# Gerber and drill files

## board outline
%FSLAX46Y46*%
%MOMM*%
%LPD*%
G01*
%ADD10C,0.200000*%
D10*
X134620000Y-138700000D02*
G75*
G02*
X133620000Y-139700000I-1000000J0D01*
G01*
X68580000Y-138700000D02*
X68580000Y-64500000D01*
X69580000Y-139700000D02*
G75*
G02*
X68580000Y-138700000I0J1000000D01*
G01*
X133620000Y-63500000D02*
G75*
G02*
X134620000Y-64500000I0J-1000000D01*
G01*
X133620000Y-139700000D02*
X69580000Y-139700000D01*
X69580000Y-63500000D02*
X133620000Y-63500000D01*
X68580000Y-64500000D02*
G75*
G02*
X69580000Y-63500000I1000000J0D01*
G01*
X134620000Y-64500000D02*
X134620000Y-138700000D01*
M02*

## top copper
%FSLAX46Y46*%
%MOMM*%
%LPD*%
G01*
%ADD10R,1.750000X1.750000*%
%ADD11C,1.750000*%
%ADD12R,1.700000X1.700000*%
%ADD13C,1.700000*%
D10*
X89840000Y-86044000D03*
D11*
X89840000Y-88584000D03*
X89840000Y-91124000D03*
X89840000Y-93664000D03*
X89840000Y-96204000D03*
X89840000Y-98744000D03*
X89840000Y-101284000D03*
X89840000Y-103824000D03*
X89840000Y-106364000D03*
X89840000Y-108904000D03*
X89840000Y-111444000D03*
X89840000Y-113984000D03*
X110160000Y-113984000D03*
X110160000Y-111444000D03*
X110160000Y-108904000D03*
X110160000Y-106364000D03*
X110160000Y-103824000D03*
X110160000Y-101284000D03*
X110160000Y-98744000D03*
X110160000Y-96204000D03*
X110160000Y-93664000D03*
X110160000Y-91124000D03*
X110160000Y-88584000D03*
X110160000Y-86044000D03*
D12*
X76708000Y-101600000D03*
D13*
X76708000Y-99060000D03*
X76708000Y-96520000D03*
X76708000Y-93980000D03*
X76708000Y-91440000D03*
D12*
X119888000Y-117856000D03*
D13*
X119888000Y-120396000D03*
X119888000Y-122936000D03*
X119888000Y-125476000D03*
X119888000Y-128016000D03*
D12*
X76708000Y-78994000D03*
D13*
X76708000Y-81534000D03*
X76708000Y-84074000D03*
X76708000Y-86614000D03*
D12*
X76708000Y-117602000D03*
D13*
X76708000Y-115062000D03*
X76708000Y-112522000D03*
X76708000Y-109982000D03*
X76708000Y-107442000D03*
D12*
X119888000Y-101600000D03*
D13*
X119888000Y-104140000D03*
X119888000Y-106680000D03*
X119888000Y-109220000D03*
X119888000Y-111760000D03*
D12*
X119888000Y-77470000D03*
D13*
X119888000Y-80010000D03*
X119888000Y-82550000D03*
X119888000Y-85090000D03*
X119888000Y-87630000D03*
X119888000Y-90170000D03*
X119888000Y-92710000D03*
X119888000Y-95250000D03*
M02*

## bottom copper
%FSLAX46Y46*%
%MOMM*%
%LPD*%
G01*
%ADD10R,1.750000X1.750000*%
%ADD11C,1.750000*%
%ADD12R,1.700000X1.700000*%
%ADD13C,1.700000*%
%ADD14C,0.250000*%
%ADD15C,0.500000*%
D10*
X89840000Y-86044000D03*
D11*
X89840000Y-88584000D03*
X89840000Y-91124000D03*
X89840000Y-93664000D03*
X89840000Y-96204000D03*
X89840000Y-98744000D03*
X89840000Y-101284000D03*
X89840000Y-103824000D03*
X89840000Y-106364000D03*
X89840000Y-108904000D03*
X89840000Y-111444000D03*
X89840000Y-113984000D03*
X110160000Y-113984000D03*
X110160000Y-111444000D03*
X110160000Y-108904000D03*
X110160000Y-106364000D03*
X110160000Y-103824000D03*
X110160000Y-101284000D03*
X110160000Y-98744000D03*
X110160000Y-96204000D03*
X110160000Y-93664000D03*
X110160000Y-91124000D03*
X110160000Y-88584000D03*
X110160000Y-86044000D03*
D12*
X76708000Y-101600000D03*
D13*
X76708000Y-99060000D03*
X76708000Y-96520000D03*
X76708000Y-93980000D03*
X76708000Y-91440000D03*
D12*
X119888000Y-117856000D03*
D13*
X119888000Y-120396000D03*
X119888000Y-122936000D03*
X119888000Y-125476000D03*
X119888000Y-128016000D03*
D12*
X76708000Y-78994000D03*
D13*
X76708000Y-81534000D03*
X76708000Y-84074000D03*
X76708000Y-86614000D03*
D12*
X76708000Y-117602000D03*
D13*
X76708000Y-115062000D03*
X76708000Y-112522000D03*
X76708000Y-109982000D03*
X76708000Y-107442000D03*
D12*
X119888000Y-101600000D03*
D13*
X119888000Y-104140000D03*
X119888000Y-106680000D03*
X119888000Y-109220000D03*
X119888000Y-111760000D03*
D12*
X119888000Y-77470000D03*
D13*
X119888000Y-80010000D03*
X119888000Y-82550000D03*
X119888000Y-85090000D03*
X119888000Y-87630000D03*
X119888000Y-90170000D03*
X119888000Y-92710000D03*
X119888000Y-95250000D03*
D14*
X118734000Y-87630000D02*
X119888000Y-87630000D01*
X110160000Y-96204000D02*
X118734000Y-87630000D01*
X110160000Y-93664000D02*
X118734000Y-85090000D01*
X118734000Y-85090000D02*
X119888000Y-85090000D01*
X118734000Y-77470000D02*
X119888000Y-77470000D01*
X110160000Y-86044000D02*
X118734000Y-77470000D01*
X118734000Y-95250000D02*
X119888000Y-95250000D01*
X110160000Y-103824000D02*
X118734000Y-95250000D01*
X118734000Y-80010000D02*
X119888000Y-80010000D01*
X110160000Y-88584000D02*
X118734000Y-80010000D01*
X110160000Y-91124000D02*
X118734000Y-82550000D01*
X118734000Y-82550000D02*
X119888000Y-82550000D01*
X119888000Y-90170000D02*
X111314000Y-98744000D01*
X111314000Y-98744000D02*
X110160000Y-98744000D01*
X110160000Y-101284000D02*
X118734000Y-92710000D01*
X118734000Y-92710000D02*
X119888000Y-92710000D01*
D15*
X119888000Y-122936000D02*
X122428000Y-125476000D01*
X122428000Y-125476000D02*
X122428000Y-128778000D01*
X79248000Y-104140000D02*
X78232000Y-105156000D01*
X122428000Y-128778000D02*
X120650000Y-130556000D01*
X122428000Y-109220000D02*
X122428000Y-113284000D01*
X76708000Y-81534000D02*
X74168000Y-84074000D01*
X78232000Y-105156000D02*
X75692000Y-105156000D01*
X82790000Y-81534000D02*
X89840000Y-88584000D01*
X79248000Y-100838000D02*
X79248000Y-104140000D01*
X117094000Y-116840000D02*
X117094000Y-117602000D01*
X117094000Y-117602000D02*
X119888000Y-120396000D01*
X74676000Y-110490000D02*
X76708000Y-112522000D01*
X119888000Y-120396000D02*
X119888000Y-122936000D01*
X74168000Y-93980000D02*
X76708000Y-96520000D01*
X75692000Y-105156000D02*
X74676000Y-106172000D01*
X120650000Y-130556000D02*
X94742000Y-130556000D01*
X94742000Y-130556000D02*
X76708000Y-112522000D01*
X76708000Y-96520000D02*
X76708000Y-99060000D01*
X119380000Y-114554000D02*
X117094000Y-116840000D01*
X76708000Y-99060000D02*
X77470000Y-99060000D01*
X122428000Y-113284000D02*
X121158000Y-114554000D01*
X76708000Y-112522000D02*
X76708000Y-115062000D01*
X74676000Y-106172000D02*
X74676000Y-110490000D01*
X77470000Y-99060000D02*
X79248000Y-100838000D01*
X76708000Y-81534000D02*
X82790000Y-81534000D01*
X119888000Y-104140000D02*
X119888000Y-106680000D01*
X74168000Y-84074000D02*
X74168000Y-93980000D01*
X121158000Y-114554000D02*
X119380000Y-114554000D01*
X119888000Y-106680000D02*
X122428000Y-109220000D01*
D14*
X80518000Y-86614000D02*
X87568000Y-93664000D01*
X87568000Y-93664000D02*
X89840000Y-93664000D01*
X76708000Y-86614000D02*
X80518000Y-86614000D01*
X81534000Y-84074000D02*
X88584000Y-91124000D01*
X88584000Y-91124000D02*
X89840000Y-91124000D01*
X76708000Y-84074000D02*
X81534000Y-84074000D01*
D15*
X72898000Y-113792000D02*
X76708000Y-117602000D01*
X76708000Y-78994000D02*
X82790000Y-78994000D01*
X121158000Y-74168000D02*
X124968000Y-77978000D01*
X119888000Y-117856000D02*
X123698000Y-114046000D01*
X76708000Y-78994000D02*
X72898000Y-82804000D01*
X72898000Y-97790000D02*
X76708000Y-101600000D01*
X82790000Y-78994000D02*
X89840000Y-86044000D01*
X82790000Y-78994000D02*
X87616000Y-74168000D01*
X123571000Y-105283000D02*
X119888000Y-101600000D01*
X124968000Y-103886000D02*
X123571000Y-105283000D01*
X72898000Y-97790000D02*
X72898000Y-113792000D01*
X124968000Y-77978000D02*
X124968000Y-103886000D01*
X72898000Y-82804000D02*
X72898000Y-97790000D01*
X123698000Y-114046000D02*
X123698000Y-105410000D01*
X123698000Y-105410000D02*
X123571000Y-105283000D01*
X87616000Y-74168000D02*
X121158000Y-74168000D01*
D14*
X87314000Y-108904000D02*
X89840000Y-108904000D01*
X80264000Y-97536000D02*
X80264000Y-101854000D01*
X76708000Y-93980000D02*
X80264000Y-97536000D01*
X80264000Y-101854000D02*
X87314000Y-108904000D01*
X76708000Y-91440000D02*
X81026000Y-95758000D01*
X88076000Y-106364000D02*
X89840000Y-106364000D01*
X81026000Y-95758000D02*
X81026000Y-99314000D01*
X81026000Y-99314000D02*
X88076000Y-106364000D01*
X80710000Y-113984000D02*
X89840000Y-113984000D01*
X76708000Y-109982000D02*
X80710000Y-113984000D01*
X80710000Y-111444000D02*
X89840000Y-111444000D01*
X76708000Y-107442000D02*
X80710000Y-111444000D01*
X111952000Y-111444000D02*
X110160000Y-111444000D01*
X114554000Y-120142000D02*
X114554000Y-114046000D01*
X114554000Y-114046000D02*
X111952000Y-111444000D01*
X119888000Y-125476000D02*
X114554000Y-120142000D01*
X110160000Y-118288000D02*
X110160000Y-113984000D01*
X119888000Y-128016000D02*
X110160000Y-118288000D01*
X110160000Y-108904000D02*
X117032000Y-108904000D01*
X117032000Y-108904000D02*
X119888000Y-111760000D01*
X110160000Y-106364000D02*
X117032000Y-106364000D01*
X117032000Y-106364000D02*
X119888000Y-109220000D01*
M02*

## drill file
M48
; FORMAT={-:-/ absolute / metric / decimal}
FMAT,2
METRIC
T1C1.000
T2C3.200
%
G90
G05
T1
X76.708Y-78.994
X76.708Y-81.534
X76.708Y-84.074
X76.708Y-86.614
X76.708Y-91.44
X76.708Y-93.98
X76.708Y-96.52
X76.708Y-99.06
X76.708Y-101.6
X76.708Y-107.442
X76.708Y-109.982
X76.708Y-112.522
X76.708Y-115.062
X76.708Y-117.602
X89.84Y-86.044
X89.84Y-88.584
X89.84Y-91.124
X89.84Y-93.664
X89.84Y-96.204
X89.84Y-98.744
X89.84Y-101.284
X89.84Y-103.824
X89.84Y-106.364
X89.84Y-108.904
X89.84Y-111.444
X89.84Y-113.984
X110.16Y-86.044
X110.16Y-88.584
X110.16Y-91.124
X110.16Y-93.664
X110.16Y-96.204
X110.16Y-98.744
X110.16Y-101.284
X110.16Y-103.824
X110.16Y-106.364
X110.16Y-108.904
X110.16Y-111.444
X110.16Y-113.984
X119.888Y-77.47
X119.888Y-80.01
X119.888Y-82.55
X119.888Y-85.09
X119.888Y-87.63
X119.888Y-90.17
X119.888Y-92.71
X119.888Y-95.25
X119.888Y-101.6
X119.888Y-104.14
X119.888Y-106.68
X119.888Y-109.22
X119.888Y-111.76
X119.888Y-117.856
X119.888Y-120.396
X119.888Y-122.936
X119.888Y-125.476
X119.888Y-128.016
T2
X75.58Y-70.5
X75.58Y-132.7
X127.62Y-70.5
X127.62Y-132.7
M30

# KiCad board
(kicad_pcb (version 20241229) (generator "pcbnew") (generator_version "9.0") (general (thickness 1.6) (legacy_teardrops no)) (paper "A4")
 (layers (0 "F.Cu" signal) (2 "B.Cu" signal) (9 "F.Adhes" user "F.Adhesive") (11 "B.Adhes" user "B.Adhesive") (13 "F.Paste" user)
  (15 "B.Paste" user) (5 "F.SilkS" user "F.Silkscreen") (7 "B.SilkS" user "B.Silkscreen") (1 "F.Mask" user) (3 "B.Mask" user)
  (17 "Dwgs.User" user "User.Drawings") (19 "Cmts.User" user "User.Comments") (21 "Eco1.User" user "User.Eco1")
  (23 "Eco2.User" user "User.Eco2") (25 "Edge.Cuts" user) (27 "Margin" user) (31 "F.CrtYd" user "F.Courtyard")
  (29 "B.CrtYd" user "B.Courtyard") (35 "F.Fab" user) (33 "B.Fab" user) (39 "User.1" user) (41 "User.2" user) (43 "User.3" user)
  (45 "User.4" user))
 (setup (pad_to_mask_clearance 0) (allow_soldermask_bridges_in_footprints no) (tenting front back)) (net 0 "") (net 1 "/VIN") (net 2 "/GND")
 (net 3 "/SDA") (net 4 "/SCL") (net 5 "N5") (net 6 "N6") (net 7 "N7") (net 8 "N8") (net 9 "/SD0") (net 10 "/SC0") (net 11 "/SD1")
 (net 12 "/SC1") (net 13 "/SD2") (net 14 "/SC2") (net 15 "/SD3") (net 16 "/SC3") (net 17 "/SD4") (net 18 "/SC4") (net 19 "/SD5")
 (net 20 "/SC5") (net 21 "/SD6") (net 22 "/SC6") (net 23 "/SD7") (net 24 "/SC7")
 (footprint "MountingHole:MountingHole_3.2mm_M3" (layer "F.Cu") (at 127.62 70.5)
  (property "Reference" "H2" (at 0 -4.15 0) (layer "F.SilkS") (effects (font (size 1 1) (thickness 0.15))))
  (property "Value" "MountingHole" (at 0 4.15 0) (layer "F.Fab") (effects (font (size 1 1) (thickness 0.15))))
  (pad "" np_thru_hole circle (at 0 0) (size 3.2 3.2) (drill 3.2) (layers "*.Cu" "*.Mask")))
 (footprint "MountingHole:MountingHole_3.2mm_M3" (layer "F.Cu") (at 127.62 132.7)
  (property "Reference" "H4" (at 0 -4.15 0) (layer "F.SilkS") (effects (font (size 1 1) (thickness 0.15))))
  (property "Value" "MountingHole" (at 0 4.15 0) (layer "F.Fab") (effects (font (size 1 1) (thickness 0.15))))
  (pad "" np_thru_hole circle (at 0 0) (size 3.2 3.2) (drill 3.2) (layers "*.Cu" "*.Mask")))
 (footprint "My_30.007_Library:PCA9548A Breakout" (layer "F.Cu") (at 89.84 86.044)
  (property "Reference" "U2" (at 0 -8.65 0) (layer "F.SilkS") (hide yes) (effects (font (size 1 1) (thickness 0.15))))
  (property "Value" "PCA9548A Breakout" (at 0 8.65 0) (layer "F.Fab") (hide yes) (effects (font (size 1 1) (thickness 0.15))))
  (pad "1" thru_hole rect (at 0 0) (size 1.75 1.75) (drill 1) (layers "*.Cu" "*.Mask") (remove_unused_layers no) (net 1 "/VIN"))
  (pad "2" thru_hole circle (at 0 2.54) (size 1.75 1.75) (drill 1) (layers "*.Cu" "*.Mask") (remove_unused_layers no) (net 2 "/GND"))
  (pad "3" thru_hole circle (at 0 5.08) (size 1.75 1.75) (drill 1) (layers "*.Cu" "*.Mask") (remove_unused_layers no) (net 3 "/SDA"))
  (pad "4" thru_hole circle (at 0 7.62) (size 1.75 1.75) (drill 1) (layers "*.Cu" "*.Mask") (remove_unused_layers no) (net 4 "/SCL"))
  (pad "5" thru_hole circle (at 0 10.16) (size 1.75 1.75) (drill 1) (layers "*.Cu" "*.Mask") (remove_unused_layers no) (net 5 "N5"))
  (pad "6" thru_hole circle (at 0 12.7) (size 1.75 1.75) (drill 1) (layers "*.Cu" "*.Mask") (remove_unused_layers no) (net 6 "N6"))
  (pad "7" thru_hole circle (at 0 15.24) (size 1.75 1.75) (drill 1) (layers "*.Cu" "*.Mask") (remove_unused_layers no) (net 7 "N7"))
  (pad "8" thru_hole circle (at 0 17.78) (size 1.75 1.75) (drill 1) (layers "*.Cu" "*.Mask") (remove_unused_layers no) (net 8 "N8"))
  (pad "9" thru_hole circle (at 0 20.32) (size 1.75 1.75) (drill 1) (layers "*.Cu" "*.Mask") (remove_unused_layers no) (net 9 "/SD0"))
  (pad "10" thru_hole circle (at 0 22.86) (size 1.75 1.75) (drill 1) (layers "*.Cu" "*.Mask") (remove_unused_layers no) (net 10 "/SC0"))
  (pad "11" thru_hole circle (at 0 25.4) (size 1.75 1.75) (drill 1) (layers "*.Cu" "*.Mask") (remove_unused_layers no) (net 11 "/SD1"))
  (pad "12" thru_hole circle (at 0 27.94) (size 1.75 1.75) (drill 1) (layers "*.Cu" "*.Mask") (remove_unused_layers no) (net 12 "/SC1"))
  (pad "13" thru_hole circle (at 20.32 27.94) (size 1.75 1.75) (drill 1) (layers "*.Cu" "*.Mask") (remove_unused_layers no) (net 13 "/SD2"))
  (pad "14" thru_hole circle (at 20.32 25.4) (size 1.75 1.75) (drill 1) (layers "*.Cu" "*.Mask") (remove_unused_layers no) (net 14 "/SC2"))
  (pad "15" thru_hole circle (at 20.32 22.86) (size 1.75 1.75) (drill 1) (layers "*.Cu" "*.Mask") (remove_unused_layers no) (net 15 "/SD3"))
  (pad "16" thru_hole circle (at 20.32 20.32) (size 1.75 1.75) (drill 1) (layers "*.Cu" "*.Mask") (remove_unused_layers no) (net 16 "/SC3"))
  (pad "17" thru_hole circle (at 20.32 17.78) (size 1.75 1.75) (drill 1) (layers "*.Cu" "*.Mask") (remove_unused_layers no) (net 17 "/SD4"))
  (pad "18" thru_hole circle (at 20.32 15.24) (size 1.75 1.75) (drill 1) (layers "*.Cu" "*.Mask") (remove_unused_layers no) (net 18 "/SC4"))
  (pad "19" thru_hole circle (at 20.32 12.7) (size 1.75 1.75) (drill 1) (layers "*.Cu" "*.Mask") (remove_unused_layers no) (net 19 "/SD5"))
  (pad "20" thru_hole circle (at 20.32 10.16) (size 1.75 1.75) (drill 1) (layers "*.Cu" "*.Mask") (remove_unused_layers no) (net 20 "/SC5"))
  (pad "21" thru_hole circle (at 20.32 7.62) (size 1.75 1.75) (drill 1) (layers "*.Cu" "*.Mask") (remove_unused_layers no) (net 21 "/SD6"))
  (pad "22" thru_hole circle (at 20.32 5.08) (size 1.75 1.75) (drill 1) (layers "*.Cu" "*.Mask") (remove_unused_layers no) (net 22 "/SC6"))
  (pad "23" thru_hole circle (at 20.32 2.54) (size 1.75 1.75) (drill 1) (layers "*.Cu" "*.Mask") (remove_unused_layers no) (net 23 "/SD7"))
  (pad "24" thru_hole circle (at 20.32 0) (size 1.75 1.75) (drill 1) (layers "*.Cu" "*.Mask") (remove_unused_layers no) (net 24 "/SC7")))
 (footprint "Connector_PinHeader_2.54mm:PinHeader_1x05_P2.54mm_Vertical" (layer "F.Cu") (at 76.708 101.6 180)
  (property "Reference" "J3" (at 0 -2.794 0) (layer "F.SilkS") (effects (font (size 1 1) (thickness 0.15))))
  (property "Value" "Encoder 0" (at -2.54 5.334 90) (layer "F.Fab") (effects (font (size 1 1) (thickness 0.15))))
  (pad "1" thru_hole rect (at 0 0 180) (size 1.7 1.7) (drill 1) (layers "*.Cu" "*.Mask") (remove_unused_layers no) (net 1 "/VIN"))
  (pad "2" thru_hole circle (at 0 2.54 180) (size 1.7 1.7) (drill 1) (layers "*.Cu" "*.Mask") (remove_unused_layers no) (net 2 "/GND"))
  (pad "3" thru_hole circle (at 0 5.08 180) (size 1.7 1.7) (drill 1) (layers "*.Cu" "*.Mask") (remove_unused_layers no) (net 2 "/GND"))
  (pad "4" thru_hole circle (at 0 7.62 180) (size 1.7 1.7) (drill 1) (layers "*.Cu" "*.Mask") (remove_unused_layers no) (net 10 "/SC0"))
  (pad "5" thru_hole circle (at 0 10.16 180) (size 1.7 1.7) (drill 1) (layers "*.Cu" "*.Mask") (remove_unused_layers no) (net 9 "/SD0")))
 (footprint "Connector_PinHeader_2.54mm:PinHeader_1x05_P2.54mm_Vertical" (layer "F.Cu") (at 119.888 117.856)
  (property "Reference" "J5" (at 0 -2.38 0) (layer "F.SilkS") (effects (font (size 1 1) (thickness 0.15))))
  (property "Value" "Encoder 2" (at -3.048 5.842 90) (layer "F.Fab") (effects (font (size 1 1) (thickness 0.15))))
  (pad "1" thru_hole rect (at 0 0) (size 1.7 1.7) (drill 1) (layers "*.Cu" "*.Mask") (remove_unused_layers no) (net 1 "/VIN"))
  (pad "2" thru_hole circle (at 0 2.54) (size 1.7 1.7) (drill 1) (layers "*.Cu" "*.Mask") (remove_unused_layers no) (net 2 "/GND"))
  (pad "3" thru_hole circle (at 0 5.08) (size 1.7 1.7) (drill 1) (layers "*.Cu" "*.Mask") (remove_unused_layers no) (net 2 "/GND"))
  (pad "4" thru_hole circle (at 0 7.62) (size 1.7 1.7) (drill 1) (layers "*.Cu" "*.Mask") (remove_unused_layers no) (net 14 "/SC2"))
  (pad "5" thru_hole circle (at 0 10.16) (size 1.7 1.7) (drill 1) (layers "*.Cu" "*.Mask") (remove_unused_layers no) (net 13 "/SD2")))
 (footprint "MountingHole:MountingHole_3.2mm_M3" (layer "F.Cu") (at 75.58 132.7)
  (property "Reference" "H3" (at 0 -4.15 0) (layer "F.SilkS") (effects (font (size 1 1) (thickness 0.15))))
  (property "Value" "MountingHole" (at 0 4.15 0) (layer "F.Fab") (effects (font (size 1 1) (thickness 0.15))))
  (pad "" np_thru_hole circle (at 0 0) (size 3.2 3.2) (drill 3.2) (layers "*.Cu" "*.Mask")))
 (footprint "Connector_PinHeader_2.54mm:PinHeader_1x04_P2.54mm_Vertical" (layer "F.Cu") (at 76.708 78.994)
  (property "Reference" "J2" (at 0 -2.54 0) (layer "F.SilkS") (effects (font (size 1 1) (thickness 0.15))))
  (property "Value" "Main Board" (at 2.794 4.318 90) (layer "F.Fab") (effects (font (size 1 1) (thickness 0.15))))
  (pad "1" thru_hole rect (at 0 0) (size 1.7 1.7) (drill 1) (layers "*.Cu" "*.Mask") (remove_unused_layers no) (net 1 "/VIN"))
  (pad "2" thru_hole circle (at 0 2.54) (size 1.7 1.7) (drill 1) (layers "*.Cu" "*.Mask") (remove_unused_layers no) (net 2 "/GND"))
  (pad "3" thru_hole circle (at 0 5.08) (size 1.7 1.7) (drill 1) (layers "*.Cu" "*.Mask") (remove_unused_layers no) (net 3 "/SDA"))
  (pad "4" thru_hole circle (at 0 7.62) (size 1.7 1.7) (drill 1) (layers "*.Cu" "*.Mask") (remove_unused_layers no) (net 4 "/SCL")))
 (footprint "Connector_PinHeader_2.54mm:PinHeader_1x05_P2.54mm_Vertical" (layer "F.Cu") (at 76.708 117.602 180)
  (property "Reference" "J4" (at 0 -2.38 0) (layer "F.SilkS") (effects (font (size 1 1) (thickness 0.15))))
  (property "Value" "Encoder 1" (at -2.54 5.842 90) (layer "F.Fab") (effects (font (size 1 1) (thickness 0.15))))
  (pad "1" thru_hole rect (at 0 0 180) (size 1.7 1.7) (drill 1) (layers "*.Cu" "*.Mask") (remove_unused_layers no) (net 1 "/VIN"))
  (pad "2" thru_hole circle (at 0 2.54 180) (size 1.7 1.7) (drill 1) (layers "*.Cu" "*.Mask") (remove_unused_layers no) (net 2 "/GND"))
  (pad "3" thru_hole circle (at 0 5.08 180) (size 1.7 1.7) (drill 1) (layers "*.Cu" "*.Mask") (remove_unused_layers no) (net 2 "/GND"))
  (pad "4" thru_hole circle (at 0 7.62 180) (size 1.7 1.7) (drill 1) (layers "*.Cu" "*.Mask") (remove_unused_layers no) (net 12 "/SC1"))
  (pad "5" thru_hole circle (at 0 10.16 180) (size 1.7 1.7) (drill 1) (layers "*.Cu" "*.Mask") (remove_unused_layers no) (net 11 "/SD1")))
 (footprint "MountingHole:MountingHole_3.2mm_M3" (layer "F.Cu") (at 75.58 70.5)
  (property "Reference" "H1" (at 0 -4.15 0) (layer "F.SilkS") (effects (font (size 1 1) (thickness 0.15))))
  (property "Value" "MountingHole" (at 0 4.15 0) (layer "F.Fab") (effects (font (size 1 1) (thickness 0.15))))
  (pad "" np_thru_hole circle (at 0 0) (size 3.2 3.2) (drill 3.2) (layers "*.Cu" "*.Mask")))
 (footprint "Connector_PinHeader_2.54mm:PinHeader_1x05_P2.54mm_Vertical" (layer "F.Cu") (at 119.888 101.6)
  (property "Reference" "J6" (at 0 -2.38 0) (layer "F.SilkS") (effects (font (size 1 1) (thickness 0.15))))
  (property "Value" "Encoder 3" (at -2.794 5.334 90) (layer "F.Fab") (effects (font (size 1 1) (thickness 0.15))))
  (pad "1" thru_hole rect (at 0 0) (size 1.7 1.7) (drill 1) (layers "*.Cu" "*.Mask") (remove_unused_layers no) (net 1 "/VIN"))
  (pad "2" thru_hole circle (at 0 2.54) (size 1.7 1.7) (drill 1) (layers "*.Cu" "*.Mask") (remove_unused_layers no) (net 2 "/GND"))
  (pad "3" thru_hole circle (at 0 5.08) (size 1.7 1.7) (drill 1) (layers "*.Cu" "*.Mask") (remove_unused_layers no) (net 2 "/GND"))
  (pad "4" thru_hole circle (at 0 7.62) (size 1.7 1.7) (drill 1) (layers "*.Cu" "*.Mask") (remove_unused_layers no) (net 16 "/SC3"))
  (pad "5" thru_hole circle (at 0 10.16) (size 1.7 1.7) (drill 1) (layers "*.Cu" "*.Mask") (remove_unused_layers no) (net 15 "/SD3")))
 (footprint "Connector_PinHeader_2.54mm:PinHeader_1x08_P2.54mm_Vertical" (layer "F.Cu") (at 119.888 77.47)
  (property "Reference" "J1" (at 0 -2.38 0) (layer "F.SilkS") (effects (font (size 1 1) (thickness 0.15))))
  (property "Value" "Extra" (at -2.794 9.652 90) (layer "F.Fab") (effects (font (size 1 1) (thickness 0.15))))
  (pad "1" thru_hole rect (at 0 0) (size 1.7 1.7) (drill 1) (layers "*.Cu" "*.Mask") (remove_unused_layers no) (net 24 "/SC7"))
  (pad "2" thru_hole circle (at 0 2.54) (size 1.7 1.7) (drill 1) (layers "*.Cu" "*.Mask") (remove_unused_layers no) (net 23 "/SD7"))
  (pad "3" thru_hole circle (at 0 5.08) (size 1.7 1.7) (drill 1) (layers "*.Cu" "*.Mask") (remove_unused_layers no) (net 22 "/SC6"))
  (pad "4" thru_hole circle (at 0 7.62) (size 1.7 1.7) (drill 1) (layers "*.Cu" "*.Mask") (remove_unused_layers no) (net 21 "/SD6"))
  (pad "5" thru_hole circle (at 0 10.16) (size 1.7 1.7) (drill 1) (layers "*.Cu" "*.Mask") (remove_unused_layers no) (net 20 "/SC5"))
  (pad "6" thru_hole circle (at 0 12.7) (size 1.7 1.7) (drill 1) (layers "*.Cu" "*.Mask") (remove_unused_layers no) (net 19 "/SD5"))
  (pad "7" thru_hole circle (at 0 15.24) (size 1.7 1.7) (drill 1) (layers "*.Cu" "*.Mask") (remove_unused_layers no) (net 18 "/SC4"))
  (pad "8" thru_hole circle (at 0 17.78) (size 1.7 1.7) (drill 1) (layers "*.Cu" "*.Mask") (remove_unused_layers no) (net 17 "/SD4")))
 (gr_arc (start 134.62 138.7) (mid 134.327107 139.407107) (end 133.62 139.7) (stroke (width 0.2) (type default)) (layer "Edge.Cuts"))
 (gr_line (start 68.58 138.7) (end 68.58 64.5) (stroke (width 0.2) (type default)) (layer "Edge.Cuts"))
 (gr_arc (start 69.58 139.7) (mid 68.872893 139.407107) (end 68.58 138.7) (stroke (width 0.2) (type default)) (layer "Edge.Cuts"))
 (gr_arc (start 133.62 63.5) (mid 134.327107 63.792893) (end 134.62 64.5) (stroke (width 0.2) (type default)) (layer "Edge.Cuts"))
 (gr_line (start 133.62 139.7) (end 69.58 139.7) (stroke (width 0.2) (type default)) (layer "Edge.Cuts"))
 (gr_line (start 69.58 63.5) (end 133.62 63.5) (stroke (width 0.2) (type default)) (layer "Edge.Cuts"))
 (gr_arc (start 68.58 64.5) (mid 68.872893 63.792893) (end 69.58 63.5) (stroke (width 0.2) (type default)) (layer "Edge.Cuts"))
 (gr_line (start 134.62 64.5) (end 134.62 138.7) (stroke (width 0.2) (type default)) (layer "Edge.Cuts"))
 (segment (start 118.734 87.63) (end 119.888 87.63) (width 0.25) (layer "B.Cu") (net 20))
 (segment (start 110.16 96.204) (end 118.734 87.63) (width 0.25) (layer "B.Cu") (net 20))
 (segment (start 110.16 93.664) (end 118.734 85.09) (width 0.25) (layer "B.Cu") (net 21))
 (segment (start 118.734 85.09) (end 119.888 85.09) (width 0.25) (layer "B.Cu") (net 21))
 (segment (start 118.734 77.47) (end 119.888 77.47) (width 0.25) (layer "B.Cu") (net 24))
 (segment (start 110.16 86.044) (end 118.734 77.47) (width 0.25) (layer "B.Cu") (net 24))
 (segment (start 118.734 95.25) (end 119.888 95.25) (width 0.25) (layer "B.Cu") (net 17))
 (segment (start 110.16 103.824) (end 118.734 95.25) (width 0.25) (layer "B.Cu") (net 17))
 (segment (start 118.734 80.01) (end 119.888 80.01) (width 0.25) (layer "B.Cu") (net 23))
 (segment (start 110.16 88.584) (end 118.734 80.01) (width 0.25) (layer "B.Cu") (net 23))
 (segment (start 110.16 91.124) (end 118.734 82.55) (width 0.25) (layer "B.Cu") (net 22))
 (segment (start 118.734 82.55) (end 119.888 82.55) (width 0.25) (layer "B.Cu") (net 22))
 (segment (start 119.888 90.17) (end 111.314 98.744) (width 0.25) (layer "B.Cu") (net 19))
 (segment (start 111.314 98.744) (end 110.16 98.744) (width 0.25) (layer "B.Cu") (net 19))
 (segment (start 110.16 101.284) (end 118.734 92.71) (width 0.25) (layer "B.Cu") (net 18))
 (segment (start 118.734 92.71) (end 119.888 92.71) (width 0.25) (layer "B.Cu") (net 18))
 (segment (start 119.888 122.936) (end 122.428 125.476) (width 0.5) (layer "B.Cu") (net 2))
 (segment (start 122.428 125.476) (end 122.428 128.778) (width 0.5) (layer "B.Cu") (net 2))
 (segment (start 79.248 104.14) (end 78.232 105.156) (width 0.5) (layer "B.Cu") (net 2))
 (segment (start 122.428 128.778) (end 120.65 130.556) (width 0.5) (layer "B.Cu") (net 2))
 (segment (start 122.428 109.22) (end 122.428 113.284) (width 0.5) (layer "B.Cu") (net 2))
 (segment (start 76.708 81.534) (end 74.168 84.074) (width 0.5) (layer "B.Cu") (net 2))
 (segment (start 78.232 105.156) (end 75.692 105.156) (width 0.5) (layer "B.Cu") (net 2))
 (segment (start 82.79 81.534) (end 89.84 88.584) (width 0.5) (layer "B.Cu") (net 2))
 (segment (start 79.248 100.838) (end 79.248 104.14) (width 0.5) (layer "B.Cu") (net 2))
 (segment (start 117.094 116.84) (end 117.094 117.602) (width 0.5) (layer "B.Cu") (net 2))
 (segment (start 117.094 117.602) (end 119.888 120.396) (width 0.5) (layer "B.Cu") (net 2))
 (segment (start 74.676 110.49) (end 76.708 112.522) (width 0.5) (layer "B.Cu") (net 2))
 (segment (start 119.888 120.396) (end 119.888 122.936) (width 0.5) (layer "B.Cu") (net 2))
 (segment (start 74.168 93.98) (end 76.708 96.52) (width 0.5) (layer "B.Cu") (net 2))
 (segment (start 75.692 105.156) (end 74.676 106.172) (width 0.5) (layer "B.Cu") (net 2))
 (segment (start 120.65 130.556) (end 94.742 130.556) (width 0.5) (layer "B.Cu") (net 2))
 (segment (start 94.742 130.556) (end 76.708 112.522) (width 0.5) (layer "B.Cu") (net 2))
 (segment (start 76.708 96.52) (end 76.708 99.06) (width 0.5) (layer "B.Cu") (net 2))
 (segment (start 119.38 114.554) (end 117.094 116.84) (width 0.5) (layer "B.Cu") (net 2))
 (segment (start 76.708 99.06) (end 77.47 99.06) (width 0.5) (layer "B.Cu") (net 2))
 (segment (start 122.428 113.284) (end 121.158 114.554) (width 0.5) (layer "B.Cu") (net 2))
 (segment (start 76.708 112.522) (end 76.708 115.062) (width 0.5) (layer "B.Cu") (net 2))
 (segment (start 74.676 106.172) (end 74.676 110.49) (width 0.5) (layer "B.Cu") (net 2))
 (segment (start 77.47 99.06) (end 79.248 100.838) (width 0.5) (layer "B.Cu") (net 2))
 (segment (start 76.708 81.534) (end 82.79 81.534) (width 0.5) (layer "B.Cu") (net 2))
 (segment (start 119.888 104.14) (end 119.888 106.68) (width 0.5) (layer "B.Cu") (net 2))
 (segment (start 74.168 84.074) (end 74.168 93.98) (width 0.5) (layer "B.Cu") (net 2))
 (segment (start 121.158 114.554) (end 119.38 114.554) (width 0.5) (layer "B.Cu") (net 2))
 (segment (start 119.888 106.68) (end 122.428 109.22) (width 0.5) (layer "B.Cu") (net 2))
 (segment (start 80.518 86.614) (end 87.568 93.664) (width 0.25) (layer "B.Cu") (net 4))
 (segment (start 87.568 93.664) (end 89.84 93.664) (width 0.25) (layer "B.Cu") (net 4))
 (segment (start 76.708 86.614) (end 80.518 86.614) (width 0.25) (layer "B.Cu") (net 4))
 (segment (start 81.534 84.074) (end 88.584 91.124) (width 0.25) (layer "B.Cu") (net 3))
 (segment (start 88.584 91.124) (end 89.84 91.124) (width 0.25) (layer "B.Cu") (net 3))
 (segment (start 76.708 84.074) (end 81.534 84.074) (width 0.25) (layer "B.Cu") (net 3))
 (segment (start 72.898 113.792) (end 76.708 117.602) (width 0.5) (layer "B.Cu") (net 1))
 (segment (start 76.708 78.994) (end 82.79 78.994) (width 0.5) (layer "B.Cu") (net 1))
 (segment (start 121.158 74.168) (end 124.968 77.978) (width 0.5) (layer "B.Cu") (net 1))
 (segment (start 119.888 117.856) (end 123.698 114.046) (width 0.5) (layer "B.Cu") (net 1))
 (segment (start 76.708 78.994) (end 72.898 82.804) (width 0.5) (layer "B.Cu") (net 1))
 (segment (start 72.898 97.79) (end 76.708 101.6) (width 0.5) (layer "B.Cu") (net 1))
 (segment (start 82.79 78.994) (end 89.84 86.044) (width 0.5) (layer "B.Cu") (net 1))
 (segment (start 82.79 78.994) (end 87.616 74.168) (width 0.5) (layer "B.Cu") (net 1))
 (segment (start 123.571 105.283) (end 119.888 101.6) (width 0.5) (layer "B.Cu") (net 1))
 (segment (start 124.968 103.886) (end 123.571 105.283) (width 0.5) (layer "B.Cu") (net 1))
 (segment (start 72.898 97.79) (end 72.898 113.792) (width 0.5) (layer "B.Cu") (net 1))
 (segment (start 124.968 77.978) (end 124.968 103.886) (width 0.5) (layer "B.Cu") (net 1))
 (segment (start 72.898 82.804) (end 72.898 97.79) (width 0.5) (layer "B.Cu") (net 1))
 (segment (start 123.698 114.046) (end 123.698 105.41) (width 0.5) (layer "B.Cu") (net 1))
 (segment (start 123.698 105.41) (end 123.571 105.283) (width 0.5) (layer "B.Cu") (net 1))
 (segment (start 87.616 74.168) (end 121.158 74.168) (width 0.5) (layer "B.Cu") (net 1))
 (segment (start 87.314 108.904) (end 89.84 108.904) (width 0.25) (layer "B.Cu") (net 10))
 (segment (start 80.264 97.536) (end 80.264 101.854) (width 0.25) (layer "B.Cu") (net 10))
 (segment (start 76.708 93.98) (end 80.264 97.536) (width 0.25) (layer "B.Cu") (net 10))
 (segment (start 80.264 101.854) (end 87.314 108.904) (width 0.25) (layer "B.Cu") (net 10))
 (segment (start 76.708 91.44) (end 81.026 95.758) (width 0.25) (layer "B.Cu") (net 9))
 (segment (start 88.076 106.364) (end 89.84 106.364) (width 0.25) (layer "B.Cu") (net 9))
 (segment (start 81.026 95.758) (end 81.026 99.314) (width 0.25) (layer "B.Cu") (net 9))
 (segment (start 81.026 99.314) (end 88.076 106.364) (width 0.25) (layer "B.Cu") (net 9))
 (segment (start 80.71 113.984) (end 89.84 113.984) (width 0.25) (layer "B.Cu") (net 12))
 (segment (start 76.708 109.982) (end 80.71 113.984) (width 0.25) (layer "B.Cu") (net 12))
 (segment (start 80.71 111.444) (end 89.84 111.444) (width 0.25) (layer "B.Cu") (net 11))
 (segment (start 76.708 107.442) (end 80.71 111.444) (width 0.25) (layer "B.Cu") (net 11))
 (segment (start 111.952 111.444) (end 110.16 111.444) (width 0.25) (layer "B.Cu") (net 14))
 (segment (start 114.554 120.142) (end 114.554 114.046) (width 0.25) (layer "B.Cu") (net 14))
 (segment (start 114.554 114.046) (end 111.952 111.444) (width 0.25) (layer "B.Cu") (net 14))
 (segment (start 119.888 125.476) (end 114.554 120.142) (width 0.25) (layer "B.Cu") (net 14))
 (segment (start 110.16 118.288) (end 110.16 113.984) (width 0.25) (layer "B.Cu") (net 13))
 (segment (start 119.888 128.016) (end 110.16 118.288) (width 0.25) (layer "B.Cu") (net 13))
 (segment (start 110.16 108.904) (end 117.032 108.904) (width 0.25) (layer "B.Cu") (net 15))
 (segment (start 117.032 108.904) (end 119.888 111.76) (width 0.25) (layer "B.Cu") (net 15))
 (segment (start 110.16 106.364) (end 117.032 106.364) (width 0.25) (layer "B.Cu") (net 16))
 (segment (start 117.032 106.364) (end 119.888 109.22) (width 0.25) (layer "B.Cu") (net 16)))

